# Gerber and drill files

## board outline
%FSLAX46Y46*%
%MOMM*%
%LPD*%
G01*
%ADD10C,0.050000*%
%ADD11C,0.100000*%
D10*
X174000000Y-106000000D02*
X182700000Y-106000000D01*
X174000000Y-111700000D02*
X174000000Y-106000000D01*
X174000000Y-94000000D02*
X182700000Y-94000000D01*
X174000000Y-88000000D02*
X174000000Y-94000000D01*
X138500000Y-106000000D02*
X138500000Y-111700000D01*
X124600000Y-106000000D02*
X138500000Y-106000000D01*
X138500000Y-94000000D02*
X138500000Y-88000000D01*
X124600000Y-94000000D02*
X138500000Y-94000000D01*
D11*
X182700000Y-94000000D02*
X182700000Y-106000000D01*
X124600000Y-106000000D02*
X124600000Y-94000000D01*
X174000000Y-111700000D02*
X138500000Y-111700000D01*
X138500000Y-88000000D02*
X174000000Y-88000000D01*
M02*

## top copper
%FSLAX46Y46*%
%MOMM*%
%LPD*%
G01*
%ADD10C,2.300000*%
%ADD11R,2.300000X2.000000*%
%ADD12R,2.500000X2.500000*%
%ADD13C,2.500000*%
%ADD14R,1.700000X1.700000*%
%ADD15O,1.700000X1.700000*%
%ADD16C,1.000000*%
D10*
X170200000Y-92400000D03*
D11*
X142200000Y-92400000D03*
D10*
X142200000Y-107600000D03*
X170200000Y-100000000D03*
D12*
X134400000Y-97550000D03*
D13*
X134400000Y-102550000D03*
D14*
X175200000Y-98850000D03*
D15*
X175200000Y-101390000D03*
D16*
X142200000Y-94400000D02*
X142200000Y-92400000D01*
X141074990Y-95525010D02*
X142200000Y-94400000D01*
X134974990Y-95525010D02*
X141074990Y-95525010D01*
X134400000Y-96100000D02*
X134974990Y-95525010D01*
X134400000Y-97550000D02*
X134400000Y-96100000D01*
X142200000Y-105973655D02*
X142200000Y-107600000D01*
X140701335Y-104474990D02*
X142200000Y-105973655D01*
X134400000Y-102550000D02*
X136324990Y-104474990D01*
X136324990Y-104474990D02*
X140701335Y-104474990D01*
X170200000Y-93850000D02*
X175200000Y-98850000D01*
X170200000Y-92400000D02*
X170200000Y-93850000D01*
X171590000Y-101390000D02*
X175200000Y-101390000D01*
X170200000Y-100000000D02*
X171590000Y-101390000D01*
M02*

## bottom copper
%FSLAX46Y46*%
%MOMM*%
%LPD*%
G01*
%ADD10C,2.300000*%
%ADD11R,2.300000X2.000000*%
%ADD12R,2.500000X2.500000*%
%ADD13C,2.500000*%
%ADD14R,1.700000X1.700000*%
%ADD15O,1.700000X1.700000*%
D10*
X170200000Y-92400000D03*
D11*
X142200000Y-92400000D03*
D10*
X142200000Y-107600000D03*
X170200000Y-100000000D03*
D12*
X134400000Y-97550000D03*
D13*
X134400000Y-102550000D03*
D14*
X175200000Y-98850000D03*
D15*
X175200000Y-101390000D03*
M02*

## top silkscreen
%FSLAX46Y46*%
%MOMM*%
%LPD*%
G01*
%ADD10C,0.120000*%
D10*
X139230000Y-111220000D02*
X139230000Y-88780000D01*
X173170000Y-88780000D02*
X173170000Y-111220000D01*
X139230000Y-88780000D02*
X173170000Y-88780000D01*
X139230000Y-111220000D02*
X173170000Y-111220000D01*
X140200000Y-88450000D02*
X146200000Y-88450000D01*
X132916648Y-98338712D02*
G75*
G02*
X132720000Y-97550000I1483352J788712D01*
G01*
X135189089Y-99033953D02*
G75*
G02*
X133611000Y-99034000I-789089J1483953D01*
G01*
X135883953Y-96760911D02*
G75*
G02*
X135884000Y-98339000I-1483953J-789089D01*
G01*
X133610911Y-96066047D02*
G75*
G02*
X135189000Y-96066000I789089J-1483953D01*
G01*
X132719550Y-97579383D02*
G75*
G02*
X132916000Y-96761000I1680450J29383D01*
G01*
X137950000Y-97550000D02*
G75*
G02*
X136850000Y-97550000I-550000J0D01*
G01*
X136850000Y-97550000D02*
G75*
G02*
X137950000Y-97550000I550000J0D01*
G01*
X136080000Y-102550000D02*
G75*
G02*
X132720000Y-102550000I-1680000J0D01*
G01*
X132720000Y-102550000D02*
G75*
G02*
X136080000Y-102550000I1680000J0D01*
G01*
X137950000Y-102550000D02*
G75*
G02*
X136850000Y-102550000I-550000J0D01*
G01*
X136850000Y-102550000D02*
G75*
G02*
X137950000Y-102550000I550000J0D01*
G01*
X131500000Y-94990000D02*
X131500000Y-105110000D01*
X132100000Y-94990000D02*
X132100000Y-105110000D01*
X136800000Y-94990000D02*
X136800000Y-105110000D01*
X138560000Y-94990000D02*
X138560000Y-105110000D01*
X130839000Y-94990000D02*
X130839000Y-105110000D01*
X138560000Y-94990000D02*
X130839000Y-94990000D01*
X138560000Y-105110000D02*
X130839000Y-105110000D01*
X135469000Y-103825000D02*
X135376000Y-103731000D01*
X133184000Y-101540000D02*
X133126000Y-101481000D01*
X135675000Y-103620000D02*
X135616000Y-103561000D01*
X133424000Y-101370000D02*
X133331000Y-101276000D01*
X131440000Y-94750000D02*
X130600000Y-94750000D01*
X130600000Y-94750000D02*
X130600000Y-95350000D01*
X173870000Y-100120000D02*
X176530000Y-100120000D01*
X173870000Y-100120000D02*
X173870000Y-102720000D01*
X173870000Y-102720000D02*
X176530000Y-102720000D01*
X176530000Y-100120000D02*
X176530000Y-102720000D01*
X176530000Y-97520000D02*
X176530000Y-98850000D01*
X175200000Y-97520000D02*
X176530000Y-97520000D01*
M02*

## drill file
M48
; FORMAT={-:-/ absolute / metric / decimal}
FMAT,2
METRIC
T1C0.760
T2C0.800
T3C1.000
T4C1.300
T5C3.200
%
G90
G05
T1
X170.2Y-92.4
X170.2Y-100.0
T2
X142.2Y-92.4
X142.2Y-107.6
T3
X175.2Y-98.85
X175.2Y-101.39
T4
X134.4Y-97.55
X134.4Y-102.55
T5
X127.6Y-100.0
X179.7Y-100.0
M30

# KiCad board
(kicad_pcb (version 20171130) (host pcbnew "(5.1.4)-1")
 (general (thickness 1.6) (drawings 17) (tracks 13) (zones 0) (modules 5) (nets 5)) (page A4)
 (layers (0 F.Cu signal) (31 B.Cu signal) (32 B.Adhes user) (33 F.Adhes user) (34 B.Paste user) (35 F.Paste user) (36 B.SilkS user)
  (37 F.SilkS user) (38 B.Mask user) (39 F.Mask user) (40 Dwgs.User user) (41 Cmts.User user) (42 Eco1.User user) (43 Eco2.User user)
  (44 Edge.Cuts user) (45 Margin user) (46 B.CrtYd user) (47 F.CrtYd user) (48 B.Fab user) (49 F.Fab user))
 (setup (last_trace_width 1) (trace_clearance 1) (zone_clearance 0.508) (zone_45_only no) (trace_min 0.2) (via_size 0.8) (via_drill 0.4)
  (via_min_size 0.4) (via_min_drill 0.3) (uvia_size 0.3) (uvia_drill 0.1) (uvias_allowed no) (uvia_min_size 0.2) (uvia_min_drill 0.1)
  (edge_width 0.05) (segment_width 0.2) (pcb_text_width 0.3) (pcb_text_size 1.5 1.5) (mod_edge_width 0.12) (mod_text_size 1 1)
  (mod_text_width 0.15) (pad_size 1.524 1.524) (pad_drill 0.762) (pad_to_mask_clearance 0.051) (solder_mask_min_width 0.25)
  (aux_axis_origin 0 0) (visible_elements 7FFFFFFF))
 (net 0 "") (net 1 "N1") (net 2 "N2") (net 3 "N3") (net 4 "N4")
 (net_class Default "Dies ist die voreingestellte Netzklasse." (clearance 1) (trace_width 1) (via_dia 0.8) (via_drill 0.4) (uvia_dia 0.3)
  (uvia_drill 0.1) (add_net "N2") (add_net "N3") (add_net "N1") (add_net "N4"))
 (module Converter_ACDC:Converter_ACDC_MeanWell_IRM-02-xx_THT (layer F.Cu) (at 142.2 92.4)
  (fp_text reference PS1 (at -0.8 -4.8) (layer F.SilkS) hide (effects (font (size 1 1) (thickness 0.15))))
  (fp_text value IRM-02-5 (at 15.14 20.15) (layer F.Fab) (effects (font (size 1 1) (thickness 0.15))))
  (fp_line (start -2.97 18.82) (end -2.97 -3.62) (layer F.SilkS) (width 0.12))
  (fp_line (start 30.97 -3.62) (end 30.97 18.82) (layer F.SilkS) (width 0.12))
  (fp_line (start -2.97 -3.62) (end 30.97 -3.62) (layer F.SilkS) (width 0.12))
  (fp_line (start -2.97 18.82) (end 30.97 18.82) (layer F.SilkS) (width 0.12))
  (fp_line (start -2 -3.95) (end 4 -3.95) (layer F.SilkS) (width 0.12))
  (pad 3 thru_hole circle (at 28 0) (size 2.3 2.3) (drill 0.76) (layers *.Cu *.Mask) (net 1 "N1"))
  (pad 1 thru_hole rect (at 0 0) (size 2.3 2) (drill 0.8) (layers *.Cu *.Mask) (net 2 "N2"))
  (pad 2 thru_hole circle (at 0 15.2) (size 2.3 2.3) (drill 0.8) (layers *.Cu *.Mask) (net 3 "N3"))
  (pad 4 thru_hole circle (at 28 7.6) (size 2.3 2.3) (drill 0.76) (layers *.Cu *.Mask) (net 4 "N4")))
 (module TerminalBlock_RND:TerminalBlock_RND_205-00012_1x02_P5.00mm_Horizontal (layer F.Cu) (at 134.4 97.55 270)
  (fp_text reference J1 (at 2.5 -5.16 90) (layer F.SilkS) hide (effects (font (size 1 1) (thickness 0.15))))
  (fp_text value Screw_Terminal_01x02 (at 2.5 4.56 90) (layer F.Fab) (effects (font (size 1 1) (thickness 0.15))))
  (fp_arc (start 0 0) (end 0 1.68) (angle -28) (layer F.SilkS) (width 0.12))
  (fp_arc (start 0 0) (end 1.484 0.789) (angle -56) (layer F.SilkS) (width 0.12))
  (fp_arc (start 0 0) (end 0.789 -1.484) (angle -56) (layer F.SilkS) (width 0.12))
  (fp_arc (start 0 0) (end -1.484 -0.789) (angle -56) (layer F.SilkS) (width 0.12))
  (fp_arc (start 0 0) (end -0.789 1.484) (angle -29) (layer F.SilkS) (width 0.12))
  (fp_circle (center 0 -3) (end 0.55 -3) (layer F.SilkS) (width 0.12))
  (fp_circle (center 5 0) (end 6.68 0) (layer F.SilkS) (width 0.12))
  (fp_circle (center 5 -3) (end 5.55 -3) (layer F.SilkS) (width 0.12))
  (fp_line (start -2.56 2.9) (end 7.56 2.9) (layer F.SilkS) (width 0.12))
  (fp_line (start -2.56 2.3) (end 7.56 2.3) (layer F.SilkS) (width 0.12))
  (fp_line (start -2.56 -2.4) (end 7.56 -2.4) (layer F.SilkS) (width 0.12))
  (fp_line (start -2.56 -4.16) (end 7.56 -4.16) (layer F.SilkS) (width 0.12))
  (fp_line (start -2.56 3.561) (end 7.56 3.561) (layer F.SilkS) (width 0.12))
  (fp_line (start -2.56 -4.16) (end -2.56 3.561) (layer F.SilkS) (width 0.12))
  (fp_line (start 7.56 -4.16) (end 7.56 3.561) (layer F.SilkS) (width 0.12))
  (fp_line (start 6.275 -1.069) (end 6.181 -0.976) (layer F.SilkS) (width 0.12))
  (fp_line (start 3.99 1.216) (end 3.931 1.274) (layer F.SilkS) (width 0.12))
  (fp_line (start 6.07 -1.275) (end 6.011 -1.216) (layer F.SilkS) (width 0.12))
  (fp_line (start 3.82 0.976) (end 3.726 1.069) (layer F.SilkS) (width 0.12))
  (fp_line (start -2.8 2.96) (end -2.8 3.8) (layer F.SilkS) (width 0.12))
  (fp_line (start -2.8 3.8) (end -2.2 3.8) (layer F.SilkS) (width 0.12))
  (pad 1 thru_hole rect (at 0 0 270) (size 2.5 2.5) (drill 1.3) (layers *.Cu *.Mask) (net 2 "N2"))
  (pad 2 thru_hole circle (at 5 0 270) (size 2.5 2.5) (drill 1.3) (layers *.Cu *.Mask) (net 3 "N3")))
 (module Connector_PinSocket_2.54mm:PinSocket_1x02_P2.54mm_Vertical (layer F.Cu) (at 175.2 98.85)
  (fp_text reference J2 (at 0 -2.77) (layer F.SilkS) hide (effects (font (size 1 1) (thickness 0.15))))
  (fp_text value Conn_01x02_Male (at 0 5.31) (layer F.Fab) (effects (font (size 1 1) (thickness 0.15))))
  (fp_line (start -1.33 1.27) (end 1.33 1.27) (layer F.SilkS) (width 0.12))
  (fp_line (start -1.33 1.27) (end -1.33 3.87) (layer F.SilkS) (width 0.12))
  (fp_line (start -1.33 3.87) (end 1.33 3.87) (layer F.SilkS) (width 0.12))
  (fp_line (start 1.33 1.27) (end 1.33 3.87) (layer F.SilkS) (width 0.12))
  (fp_line (start 1.33 -1.33) (end 1.33 0) (layer F.SilkS) (width 0.12))
  (fp_line (start 0 -1.33) (end 1.33 -1.33) (layer F.SilkS) (width 0.12))
  (pad 1 thru_hole rect (at 0 0) (size 1.7 1.7) (drill 1) (layers *.Cu *.Mask) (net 1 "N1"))
  (pad 2 thru_hole oval (at 0 2.54) (size 1.7 1.7) (drill 1) (layers *.Cu *.Mask) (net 4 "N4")))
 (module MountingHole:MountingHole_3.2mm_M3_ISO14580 (layer F.Cu) (at 127.6 100)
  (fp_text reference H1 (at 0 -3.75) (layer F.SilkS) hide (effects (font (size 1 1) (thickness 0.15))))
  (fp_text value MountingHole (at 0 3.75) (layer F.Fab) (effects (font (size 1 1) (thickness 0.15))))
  (pad 1 np_thru_hole circle (at 0 0) (size 3.2 3.2) (drill 3.2) (layers *.Cu *.Mask)))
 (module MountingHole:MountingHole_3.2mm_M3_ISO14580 (layer F.Cu) (at 179.7 100)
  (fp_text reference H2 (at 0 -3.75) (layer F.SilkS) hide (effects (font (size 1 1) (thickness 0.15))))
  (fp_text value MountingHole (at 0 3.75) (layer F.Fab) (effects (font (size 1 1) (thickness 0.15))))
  (pad 1 np_thru_hole circle (at 0 0) (size 3.2 3.2) (drill 3.2) (layers *.Cu *.Mask)))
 (gr_line (start 174 106) (end 182.7 106) (layer Edge.Cuts) (width 0.05))
 (gr_line (start 174 111.7) (end 174 106) (layer Edge.Cuts) (width 0.05))
 (gr_line (start 174 94) (end 182.7 94) (layer Edge.Cuts) (width 0.05))
 (gr_line (start 174 88) (end 174 94) (layer Edge.Cuts) (width 0.05))
 (gr_line (start 138.5 106) (end 138.5 111.7) (layer Edge.Cuts) (width 0.05))
 (gr_line (start 124.6 106) (end 138.5 106) (layer Edge.Cuts) (width 0.05))
 (gr_line (start 138.5 94) (end 138.5 88) (layer Edge.Cuts) (width 0.05))
 (gr_line (start 124.6 94) (end 138.5 94) (layer Edge.Cuts) (width 0.05))
 (gr_line (start 182.7 94) (end 182.7 106) (layer Edge.Cuts) (width 0.1))
 (gr_line (start 124.6 106) (end 124.6 94) (layer Edge.Cuts) (width 0.1))
 (gr_line (start 174 111.7) (end 138.5 111.7) (layer Edge.Cuts) (width 0.1))
 (gr_line (start 138.5 88) (end 174 88) (layer Edge.Cuts) (width 0.1))
 (segment (start 142.2 94.4) (end 142.2 92.4) (width 1) (layer F.Cu) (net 2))
 (segment (start 141.07499 95.52501) (end 142.2 94.4) (width 1) (layer F.Cu) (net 2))
 (segment (start 134.97499 95.52501) (end 141.07499 95.52501) (width 1) (layer F.Cu) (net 2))
 (segment (start 134.4 96.1) (end 134.97499 95.52501) (width 1) (layer F.Cu) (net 2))
 (segment (start 134.4 97.55) (end 134.4 96.1) (width 1) (layer F.Cu) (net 2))
 (segment (start 142.2 105.973655) (end 142.2 107.6) (width 1) (layer F.Cu) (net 3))
 (segment (start 140.701335 104.47499) (end 142.2 105.973655) (width 1) (layer F.Cu) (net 3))
 (segment (start 134.4 102.55) (end 136.32499 104.47499) (width 1) (layer F.Cu) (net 3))
 (segment (start 136.32499 104.47499) (end 140.701335 104.47499) (width 1) (layer F.Cu) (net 3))
 (segment (start 170.2 93.85) (end 175.2 98.85) (width 1) (layer F.Cu) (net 1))
 (segment (start 170.2 92.4) (end 170.2 93.85) (width 1) (layer F.Cu) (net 1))
 (segment (start 171.59 101.39) (end 175.2 101.39) (width 1) (layer F.Cu) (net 4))
 (segment (start 170.2 100) (end 171.59 101.39) (width 1) (layer F.Cu) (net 4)))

